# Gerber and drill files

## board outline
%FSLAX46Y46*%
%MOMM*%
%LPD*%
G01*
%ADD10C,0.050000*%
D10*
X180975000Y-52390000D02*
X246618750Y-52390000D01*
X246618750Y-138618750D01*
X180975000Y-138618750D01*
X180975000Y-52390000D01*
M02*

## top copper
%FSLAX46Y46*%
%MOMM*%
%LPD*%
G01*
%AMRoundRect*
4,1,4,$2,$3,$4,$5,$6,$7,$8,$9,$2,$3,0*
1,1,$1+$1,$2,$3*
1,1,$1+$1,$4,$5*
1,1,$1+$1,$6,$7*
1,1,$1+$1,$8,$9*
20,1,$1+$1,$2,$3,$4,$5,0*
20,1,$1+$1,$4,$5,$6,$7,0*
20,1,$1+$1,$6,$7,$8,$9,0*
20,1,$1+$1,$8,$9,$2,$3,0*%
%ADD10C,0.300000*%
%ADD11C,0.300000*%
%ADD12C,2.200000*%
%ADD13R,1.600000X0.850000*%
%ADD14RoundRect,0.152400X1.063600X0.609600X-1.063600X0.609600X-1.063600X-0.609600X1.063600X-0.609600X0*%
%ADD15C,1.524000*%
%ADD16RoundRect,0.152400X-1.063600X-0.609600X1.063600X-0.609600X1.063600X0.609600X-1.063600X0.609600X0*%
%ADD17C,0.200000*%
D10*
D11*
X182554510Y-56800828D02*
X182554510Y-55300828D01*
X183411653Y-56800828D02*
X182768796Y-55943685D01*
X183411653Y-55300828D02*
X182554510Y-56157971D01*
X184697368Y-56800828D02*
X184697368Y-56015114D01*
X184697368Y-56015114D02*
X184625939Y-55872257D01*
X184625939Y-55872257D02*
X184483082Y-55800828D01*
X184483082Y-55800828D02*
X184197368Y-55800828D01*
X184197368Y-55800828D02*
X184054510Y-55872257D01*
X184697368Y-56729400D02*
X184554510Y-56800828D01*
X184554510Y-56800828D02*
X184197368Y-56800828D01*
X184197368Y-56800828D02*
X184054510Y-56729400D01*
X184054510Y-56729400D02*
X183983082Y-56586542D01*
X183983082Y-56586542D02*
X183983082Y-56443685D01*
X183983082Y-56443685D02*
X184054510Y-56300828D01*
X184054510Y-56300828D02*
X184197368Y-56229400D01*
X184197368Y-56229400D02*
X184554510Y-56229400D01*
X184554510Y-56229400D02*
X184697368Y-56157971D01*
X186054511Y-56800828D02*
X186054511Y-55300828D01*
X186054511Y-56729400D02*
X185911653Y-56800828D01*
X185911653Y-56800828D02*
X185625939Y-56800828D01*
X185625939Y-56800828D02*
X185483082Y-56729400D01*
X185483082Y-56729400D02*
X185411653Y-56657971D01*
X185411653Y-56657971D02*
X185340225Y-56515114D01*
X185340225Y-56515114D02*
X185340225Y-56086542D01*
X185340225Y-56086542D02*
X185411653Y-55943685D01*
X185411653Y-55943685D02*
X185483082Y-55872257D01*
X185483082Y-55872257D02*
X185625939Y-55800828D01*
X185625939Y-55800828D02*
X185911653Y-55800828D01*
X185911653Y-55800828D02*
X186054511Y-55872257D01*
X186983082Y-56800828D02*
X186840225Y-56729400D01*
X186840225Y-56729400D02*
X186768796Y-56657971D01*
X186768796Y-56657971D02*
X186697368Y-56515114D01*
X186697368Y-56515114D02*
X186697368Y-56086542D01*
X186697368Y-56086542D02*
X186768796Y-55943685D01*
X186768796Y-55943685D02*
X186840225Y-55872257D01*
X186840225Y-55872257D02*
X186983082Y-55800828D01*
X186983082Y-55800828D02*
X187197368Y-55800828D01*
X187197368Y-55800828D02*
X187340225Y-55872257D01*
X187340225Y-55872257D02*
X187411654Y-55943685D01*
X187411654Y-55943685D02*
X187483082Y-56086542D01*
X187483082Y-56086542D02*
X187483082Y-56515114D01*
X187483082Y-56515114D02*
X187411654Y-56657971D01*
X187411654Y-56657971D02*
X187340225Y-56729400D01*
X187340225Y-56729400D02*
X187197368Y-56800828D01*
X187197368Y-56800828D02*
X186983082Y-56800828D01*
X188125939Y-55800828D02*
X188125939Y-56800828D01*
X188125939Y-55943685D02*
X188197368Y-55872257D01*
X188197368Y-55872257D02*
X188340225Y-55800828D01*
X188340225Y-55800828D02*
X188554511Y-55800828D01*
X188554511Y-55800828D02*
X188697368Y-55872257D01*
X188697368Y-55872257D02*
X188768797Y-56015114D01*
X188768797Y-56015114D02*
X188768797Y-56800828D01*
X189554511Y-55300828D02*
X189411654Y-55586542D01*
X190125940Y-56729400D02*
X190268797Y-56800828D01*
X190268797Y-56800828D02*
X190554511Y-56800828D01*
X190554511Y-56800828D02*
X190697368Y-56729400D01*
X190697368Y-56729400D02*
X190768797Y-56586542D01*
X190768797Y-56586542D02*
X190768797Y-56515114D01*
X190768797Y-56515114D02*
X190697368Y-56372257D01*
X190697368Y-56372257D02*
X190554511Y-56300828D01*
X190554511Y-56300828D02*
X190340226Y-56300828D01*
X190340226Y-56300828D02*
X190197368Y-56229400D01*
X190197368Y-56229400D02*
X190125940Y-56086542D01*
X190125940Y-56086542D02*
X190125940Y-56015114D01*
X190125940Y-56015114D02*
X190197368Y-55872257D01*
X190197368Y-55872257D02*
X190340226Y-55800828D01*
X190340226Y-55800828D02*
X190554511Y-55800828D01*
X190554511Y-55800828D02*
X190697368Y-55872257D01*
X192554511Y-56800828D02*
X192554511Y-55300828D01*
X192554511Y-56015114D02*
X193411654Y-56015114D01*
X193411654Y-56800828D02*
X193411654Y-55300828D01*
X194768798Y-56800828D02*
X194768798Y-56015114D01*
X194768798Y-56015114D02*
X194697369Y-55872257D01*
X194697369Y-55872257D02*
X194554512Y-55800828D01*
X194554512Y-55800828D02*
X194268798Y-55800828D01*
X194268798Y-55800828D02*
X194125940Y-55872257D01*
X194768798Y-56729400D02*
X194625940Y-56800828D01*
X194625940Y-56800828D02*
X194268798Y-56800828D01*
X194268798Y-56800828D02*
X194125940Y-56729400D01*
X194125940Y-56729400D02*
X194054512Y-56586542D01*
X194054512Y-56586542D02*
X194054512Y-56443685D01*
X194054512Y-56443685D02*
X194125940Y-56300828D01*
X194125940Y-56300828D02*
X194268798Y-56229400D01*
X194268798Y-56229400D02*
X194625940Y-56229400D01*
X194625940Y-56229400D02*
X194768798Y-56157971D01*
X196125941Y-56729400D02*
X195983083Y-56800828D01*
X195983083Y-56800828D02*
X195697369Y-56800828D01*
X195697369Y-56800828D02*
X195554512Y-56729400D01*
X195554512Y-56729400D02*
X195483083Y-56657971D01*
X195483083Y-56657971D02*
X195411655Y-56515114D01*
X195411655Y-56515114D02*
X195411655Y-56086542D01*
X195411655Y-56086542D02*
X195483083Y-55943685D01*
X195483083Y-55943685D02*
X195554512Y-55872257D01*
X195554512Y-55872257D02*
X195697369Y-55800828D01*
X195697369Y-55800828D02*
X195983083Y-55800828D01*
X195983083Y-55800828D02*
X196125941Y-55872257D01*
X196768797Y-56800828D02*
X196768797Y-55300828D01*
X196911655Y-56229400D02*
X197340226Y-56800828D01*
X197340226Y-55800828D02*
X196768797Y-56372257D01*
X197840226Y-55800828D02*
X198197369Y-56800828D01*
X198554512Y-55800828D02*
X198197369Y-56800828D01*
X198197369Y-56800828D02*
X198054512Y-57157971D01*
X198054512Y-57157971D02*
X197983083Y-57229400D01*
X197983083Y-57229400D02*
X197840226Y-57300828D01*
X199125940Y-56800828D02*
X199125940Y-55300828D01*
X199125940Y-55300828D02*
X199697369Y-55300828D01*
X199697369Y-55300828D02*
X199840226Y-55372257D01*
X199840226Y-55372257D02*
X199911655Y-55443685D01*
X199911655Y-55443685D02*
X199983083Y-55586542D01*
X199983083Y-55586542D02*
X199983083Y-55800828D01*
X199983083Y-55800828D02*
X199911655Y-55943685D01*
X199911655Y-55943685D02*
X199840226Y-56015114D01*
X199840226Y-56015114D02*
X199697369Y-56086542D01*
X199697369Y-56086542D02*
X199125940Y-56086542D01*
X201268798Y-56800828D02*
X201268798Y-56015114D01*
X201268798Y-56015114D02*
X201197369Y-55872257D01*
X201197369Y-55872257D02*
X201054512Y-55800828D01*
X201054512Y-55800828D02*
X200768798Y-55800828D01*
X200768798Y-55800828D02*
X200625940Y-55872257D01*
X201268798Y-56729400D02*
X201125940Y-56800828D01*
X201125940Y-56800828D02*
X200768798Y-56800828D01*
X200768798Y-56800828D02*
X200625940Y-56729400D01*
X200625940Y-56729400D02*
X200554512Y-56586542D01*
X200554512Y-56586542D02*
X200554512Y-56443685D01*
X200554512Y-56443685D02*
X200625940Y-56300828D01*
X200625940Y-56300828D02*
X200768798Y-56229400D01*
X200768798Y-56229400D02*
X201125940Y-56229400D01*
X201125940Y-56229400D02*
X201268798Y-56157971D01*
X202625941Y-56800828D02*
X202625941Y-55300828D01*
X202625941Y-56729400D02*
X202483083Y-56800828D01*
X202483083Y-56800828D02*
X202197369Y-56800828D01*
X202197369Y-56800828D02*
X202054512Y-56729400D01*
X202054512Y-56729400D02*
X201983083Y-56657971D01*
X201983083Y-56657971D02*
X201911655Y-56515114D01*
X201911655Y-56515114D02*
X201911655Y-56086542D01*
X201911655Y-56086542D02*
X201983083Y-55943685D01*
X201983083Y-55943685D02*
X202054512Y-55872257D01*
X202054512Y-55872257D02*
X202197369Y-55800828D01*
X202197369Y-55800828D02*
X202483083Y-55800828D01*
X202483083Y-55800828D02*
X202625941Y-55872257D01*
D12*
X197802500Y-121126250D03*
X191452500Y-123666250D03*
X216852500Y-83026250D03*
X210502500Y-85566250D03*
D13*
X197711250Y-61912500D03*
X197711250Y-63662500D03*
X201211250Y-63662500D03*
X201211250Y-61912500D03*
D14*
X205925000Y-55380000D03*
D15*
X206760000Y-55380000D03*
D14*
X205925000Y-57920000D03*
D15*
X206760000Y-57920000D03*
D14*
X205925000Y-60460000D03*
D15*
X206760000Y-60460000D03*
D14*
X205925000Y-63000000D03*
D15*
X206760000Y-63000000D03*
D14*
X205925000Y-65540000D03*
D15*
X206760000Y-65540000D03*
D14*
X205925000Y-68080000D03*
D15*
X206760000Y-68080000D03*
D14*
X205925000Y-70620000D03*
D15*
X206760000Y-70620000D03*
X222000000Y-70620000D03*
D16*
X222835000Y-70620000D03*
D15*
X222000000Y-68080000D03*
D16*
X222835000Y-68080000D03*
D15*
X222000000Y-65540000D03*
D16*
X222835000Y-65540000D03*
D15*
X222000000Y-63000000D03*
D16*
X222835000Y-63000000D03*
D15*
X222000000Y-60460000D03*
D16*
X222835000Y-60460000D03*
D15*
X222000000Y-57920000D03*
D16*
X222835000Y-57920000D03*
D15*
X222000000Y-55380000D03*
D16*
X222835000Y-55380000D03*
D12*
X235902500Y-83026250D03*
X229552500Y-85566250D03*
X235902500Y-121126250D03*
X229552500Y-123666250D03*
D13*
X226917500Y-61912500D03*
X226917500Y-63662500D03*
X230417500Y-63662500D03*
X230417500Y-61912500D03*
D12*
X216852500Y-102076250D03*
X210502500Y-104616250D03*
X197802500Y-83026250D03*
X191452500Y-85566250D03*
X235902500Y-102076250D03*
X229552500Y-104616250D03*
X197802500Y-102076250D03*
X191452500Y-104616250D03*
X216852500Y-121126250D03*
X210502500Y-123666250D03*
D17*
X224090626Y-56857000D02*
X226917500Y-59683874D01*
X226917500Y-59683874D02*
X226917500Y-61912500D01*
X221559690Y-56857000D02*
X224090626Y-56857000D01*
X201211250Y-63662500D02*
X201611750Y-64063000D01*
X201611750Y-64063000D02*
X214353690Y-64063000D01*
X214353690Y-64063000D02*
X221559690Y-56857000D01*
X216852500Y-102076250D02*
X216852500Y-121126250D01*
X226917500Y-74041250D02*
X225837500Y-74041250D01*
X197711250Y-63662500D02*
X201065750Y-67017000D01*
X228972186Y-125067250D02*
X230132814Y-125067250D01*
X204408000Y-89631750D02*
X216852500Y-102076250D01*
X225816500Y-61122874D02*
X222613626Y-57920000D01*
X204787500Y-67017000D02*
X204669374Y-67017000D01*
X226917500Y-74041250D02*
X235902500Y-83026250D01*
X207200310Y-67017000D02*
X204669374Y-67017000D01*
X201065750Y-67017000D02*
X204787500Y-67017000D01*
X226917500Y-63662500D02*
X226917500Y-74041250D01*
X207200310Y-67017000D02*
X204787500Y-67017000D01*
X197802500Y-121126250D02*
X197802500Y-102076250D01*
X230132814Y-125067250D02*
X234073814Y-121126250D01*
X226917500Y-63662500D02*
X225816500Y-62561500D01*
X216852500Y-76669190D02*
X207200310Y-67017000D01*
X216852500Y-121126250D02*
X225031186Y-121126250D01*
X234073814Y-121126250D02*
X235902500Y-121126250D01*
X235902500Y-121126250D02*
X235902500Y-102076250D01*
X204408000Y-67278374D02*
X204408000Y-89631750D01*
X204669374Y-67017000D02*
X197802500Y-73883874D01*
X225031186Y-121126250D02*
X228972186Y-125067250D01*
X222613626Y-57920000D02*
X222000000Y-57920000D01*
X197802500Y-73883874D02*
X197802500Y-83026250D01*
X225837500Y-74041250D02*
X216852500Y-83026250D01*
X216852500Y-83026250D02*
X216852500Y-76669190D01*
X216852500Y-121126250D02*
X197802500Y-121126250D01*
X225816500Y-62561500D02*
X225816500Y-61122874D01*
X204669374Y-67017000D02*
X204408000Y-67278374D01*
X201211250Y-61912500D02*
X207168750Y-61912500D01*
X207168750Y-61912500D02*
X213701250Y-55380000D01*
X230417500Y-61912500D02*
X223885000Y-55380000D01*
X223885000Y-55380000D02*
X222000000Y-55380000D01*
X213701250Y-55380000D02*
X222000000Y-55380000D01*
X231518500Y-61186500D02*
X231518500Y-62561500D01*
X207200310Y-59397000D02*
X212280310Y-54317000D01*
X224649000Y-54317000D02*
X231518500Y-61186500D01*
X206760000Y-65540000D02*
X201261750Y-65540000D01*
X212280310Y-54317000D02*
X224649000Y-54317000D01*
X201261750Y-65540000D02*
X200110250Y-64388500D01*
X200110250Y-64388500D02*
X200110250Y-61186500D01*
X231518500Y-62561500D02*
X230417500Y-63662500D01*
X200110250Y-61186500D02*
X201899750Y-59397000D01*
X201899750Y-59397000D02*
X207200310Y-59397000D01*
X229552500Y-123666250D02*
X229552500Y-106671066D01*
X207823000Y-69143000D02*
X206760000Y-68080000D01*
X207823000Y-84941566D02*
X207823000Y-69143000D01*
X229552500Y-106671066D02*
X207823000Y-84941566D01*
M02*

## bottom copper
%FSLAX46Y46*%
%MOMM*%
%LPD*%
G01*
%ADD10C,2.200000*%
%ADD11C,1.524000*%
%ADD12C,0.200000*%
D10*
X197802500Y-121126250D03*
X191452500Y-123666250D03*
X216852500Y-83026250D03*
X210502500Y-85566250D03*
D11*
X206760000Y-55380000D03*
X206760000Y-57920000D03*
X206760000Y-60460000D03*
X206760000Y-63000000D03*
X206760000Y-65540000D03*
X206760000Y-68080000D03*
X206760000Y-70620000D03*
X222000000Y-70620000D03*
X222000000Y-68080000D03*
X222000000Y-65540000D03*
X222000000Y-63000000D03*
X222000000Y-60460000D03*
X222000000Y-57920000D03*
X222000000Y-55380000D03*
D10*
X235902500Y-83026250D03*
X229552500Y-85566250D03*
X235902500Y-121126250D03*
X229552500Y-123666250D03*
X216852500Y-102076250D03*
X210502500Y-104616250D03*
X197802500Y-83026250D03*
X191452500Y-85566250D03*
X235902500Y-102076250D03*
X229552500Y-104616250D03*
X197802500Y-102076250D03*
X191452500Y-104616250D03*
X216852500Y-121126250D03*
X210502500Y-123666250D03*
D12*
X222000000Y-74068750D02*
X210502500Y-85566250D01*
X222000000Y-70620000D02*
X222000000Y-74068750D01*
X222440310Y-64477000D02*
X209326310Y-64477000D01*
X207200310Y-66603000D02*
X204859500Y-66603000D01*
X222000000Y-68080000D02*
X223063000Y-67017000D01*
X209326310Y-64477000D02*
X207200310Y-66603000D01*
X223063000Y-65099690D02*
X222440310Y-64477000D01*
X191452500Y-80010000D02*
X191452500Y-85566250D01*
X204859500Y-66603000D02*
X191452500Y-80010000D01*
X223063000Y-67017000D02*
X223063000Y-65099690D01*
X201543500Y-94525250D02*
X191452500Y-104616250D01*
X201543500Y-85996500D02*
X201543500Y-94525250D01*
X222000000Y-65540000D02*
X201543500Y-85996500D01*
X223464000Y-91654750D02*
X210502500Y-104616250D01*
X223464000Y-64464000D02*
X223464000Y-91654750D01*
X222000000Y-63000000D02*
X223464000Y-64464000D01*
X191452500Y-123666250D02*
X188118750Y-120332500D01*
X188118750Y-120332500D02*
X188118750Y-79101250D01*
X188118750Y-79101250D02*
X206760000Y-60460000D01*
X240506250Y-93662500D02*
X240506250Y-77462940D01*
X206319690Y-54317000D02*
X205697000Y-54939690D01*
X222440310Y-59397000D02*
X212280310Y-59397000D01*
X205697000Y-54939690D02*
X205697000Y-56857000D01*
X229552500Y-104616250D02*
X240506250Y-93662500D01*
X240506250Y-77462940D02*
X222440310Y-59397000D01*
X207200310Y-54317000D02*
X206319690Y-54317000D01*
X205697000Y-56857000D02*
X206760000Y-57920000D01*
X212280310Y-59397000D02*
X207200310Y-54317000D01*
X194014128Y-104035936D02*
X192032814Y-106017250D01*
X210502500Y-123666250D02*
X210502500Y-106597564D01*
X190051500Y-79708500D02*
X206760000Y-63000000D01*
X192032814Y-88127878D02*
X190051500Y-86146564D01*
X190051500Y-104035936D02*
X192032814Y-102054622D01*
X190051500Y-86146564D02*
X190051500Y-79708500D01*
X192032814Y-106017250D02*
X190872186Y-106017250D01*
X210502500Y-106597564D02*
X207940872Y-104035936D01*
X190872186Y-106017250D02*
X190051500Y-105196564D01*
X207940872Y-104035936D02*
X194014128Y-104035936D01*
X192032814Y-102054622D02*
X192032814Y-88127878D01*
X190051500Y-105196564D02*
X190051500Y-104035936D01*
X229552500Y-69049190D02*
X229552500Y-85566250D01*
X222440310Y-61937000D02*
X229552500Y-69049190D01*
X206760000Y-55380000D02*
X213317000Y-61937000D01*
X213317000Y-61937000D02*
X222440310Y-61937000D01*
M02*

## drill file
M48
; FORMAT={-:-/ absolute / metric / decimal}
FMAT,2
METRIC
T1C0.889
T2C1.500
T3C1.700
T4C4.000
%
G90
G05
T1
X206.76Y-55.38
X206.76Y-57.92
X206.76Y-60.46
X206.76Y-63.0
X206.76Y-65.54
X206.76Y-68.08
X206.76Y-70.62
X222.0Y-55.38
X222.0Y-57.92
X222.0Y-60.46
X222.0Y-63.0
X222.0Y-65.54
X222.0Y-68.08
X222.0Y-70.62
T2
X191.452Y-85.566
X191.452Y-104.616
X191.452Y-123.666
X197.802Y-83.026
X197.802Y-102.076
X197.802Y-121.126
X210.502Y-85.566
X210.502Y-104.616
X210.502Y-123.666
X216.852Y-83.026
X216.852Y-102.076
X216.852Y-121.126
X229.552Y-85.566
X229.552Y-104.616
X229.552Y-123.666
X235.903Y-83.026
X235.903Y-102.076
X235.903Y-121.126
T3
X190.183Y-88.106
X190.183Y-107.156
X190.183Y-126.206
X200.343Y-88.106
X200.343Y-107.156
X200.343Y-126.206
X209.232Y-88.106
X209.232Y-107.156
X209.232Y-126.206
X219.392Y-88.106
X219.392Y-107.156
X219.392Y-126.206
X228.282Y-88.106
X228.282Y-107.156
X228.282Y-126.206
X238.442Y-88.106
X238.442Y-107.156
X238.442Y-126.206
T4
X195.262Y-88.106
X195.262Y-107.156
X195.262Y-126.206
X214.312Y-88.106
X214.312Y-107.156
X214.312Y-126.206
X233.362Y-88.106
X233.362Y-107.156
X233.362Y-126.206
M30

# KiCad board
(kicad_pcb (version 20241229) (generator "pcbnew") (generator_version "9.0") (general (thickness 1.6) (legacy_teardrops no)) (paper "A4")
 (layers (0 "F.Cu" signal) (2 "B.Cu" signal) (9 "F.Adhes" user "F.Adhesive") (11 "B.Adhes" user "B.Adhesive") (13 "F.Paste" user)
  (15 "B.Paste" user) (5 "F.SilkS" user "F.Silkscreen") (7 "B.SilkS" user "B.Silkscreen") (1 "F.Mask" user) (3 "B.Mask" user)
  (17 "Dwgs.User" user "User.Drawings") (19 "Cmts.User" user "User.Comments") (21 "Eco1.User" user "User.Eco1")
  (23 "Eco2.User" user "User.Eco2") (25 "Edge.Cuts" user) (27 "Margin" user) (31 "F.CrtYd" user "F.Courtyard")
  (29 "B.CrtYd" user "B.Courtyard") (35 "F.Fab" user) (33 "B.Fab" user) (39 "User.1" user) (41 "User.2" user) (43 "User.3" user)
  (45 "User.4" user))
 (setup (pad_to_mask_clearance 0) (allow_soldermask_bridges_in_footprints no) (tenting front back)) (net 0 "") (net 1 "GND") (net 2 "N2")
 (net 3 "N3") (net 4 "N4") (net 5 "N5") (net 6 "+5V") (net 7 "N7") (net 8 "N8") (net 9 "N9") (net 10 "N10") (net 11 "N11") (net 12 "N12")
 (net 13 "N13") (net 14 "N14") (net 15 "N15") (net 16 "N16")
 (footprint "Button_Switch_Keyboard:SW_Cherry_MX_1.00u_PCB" (layer "F.Cu") (at 197.8025 121.12625)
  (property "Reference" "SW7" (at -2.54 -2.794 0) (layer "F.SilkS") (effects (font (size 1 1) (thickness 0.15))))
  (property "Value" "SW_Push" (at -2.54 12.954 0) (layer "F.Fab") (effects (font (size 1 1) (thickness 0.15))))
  (pad "" np_thru_hole circle (at -7.62 5.08) (size 1.7 1.7) (drill 1.7) (layers "*.Cu" "*.Mask"))
  (pad "" np_thru_hole circle (at -2.54 5.08) (size 4 4) (drill 4) (layers "*.Cu" "*.Mask"))
  (pad "" np_thru_hole circle (at 2.54 5.08) (size 1.7 1.7) (drill 1.7) (layers "*.Cu" "*.Mask"))
  (pad "1" thru_hole circle (at 0 0) (size 2.2 2.2) (drill 1.5) (layers "*.Cu" "*.Mask") (remove_unused_layers no) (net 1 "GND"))
  (pad "2" thru_hole circle (at -6.35 2.54) (size 2.2 2.2) (drill 1.5) (layers "*.Cu" "*.Mask") (remove_unused_layers no) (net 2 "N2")))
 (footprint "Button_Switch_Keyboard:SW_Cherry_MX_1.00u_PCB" (layer "F.Cu") (at 216.8525 83.02625)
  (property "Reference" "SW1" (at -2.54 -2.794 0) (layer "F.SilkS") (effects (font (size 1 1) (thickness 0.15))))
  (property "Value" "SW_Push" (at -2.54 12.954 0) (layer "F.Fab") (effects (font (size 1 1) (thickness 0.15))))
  (pad "" np_thru_hole circle (at -7.62 5.08) (size 1.7 1.7) (drill 1.7) (layers "*.Cu" "*.Mask"))
  (pad "" np_thru_hole circle (at -2.54 5.08) (size 4 4) (drill 4) (layers "*.Cu" "*.Mask"))
  (pad "" np_thru_hole circle (at 2.54 5.08) (size 1.7 1.7) (drill 1.7) (layers "*.Cu" "*.Mask"))
  (pad "1" thru_hole circle (at 0 0) (size 2.2 2.2) (drill 1.5) (layers "*.Cu" "*.Mask") (remove_unused_layers no) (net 1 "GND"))
  (pad "2" thru_hole circle (at -6.35 2.54) (size 2.2 2.2) (drill 1.5) (layers "*.Cu" "*.Mask") (remove_unused_layers no) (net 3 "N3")))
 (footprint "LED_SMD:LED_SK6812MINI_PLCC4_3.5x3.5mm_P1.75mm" (layer "F.Cu") (at 199.46125 62.7875)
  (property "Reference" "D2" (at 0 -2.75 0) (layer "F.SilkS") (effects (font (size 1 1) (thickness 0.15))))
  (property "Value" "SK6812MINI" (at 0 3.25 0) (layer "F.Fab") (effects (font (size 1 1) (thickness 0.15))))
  (pad "1" smd rect (at -1.75 -0.875) (size 1.6 0.85) (layers "F.Cu" "F.Mask" "F.Paste") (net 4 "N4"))
  (pad "2" smd rect (at -1.75 0.875) (size 1.6 0.85) (layers "F.Cu" "F.Mask" "F.Paste") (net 1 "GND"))
  (pad "3" smd rect (at 1.75 0.875) (size 1.6 0.85) (layers "F.Cu" "F.Mask" "F.Paste") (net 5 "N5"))
  (pad "4" smd rect (at 1.75 -0.875) (size 1.6 0.85) (layers "F.Cu" "F.Mask" "F.Paste") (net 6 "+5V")))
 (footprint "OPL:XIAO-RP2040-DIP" (layer "F.Cu") (at 214.38 63)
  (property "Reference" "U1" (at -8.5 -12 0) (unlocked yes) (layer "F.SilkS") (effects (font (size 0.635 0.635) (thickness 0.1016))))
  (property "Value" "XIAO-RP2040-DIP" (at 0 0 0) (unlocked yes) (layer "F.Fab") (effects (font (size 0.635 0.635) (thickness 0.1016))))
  (pad "1" smd roundrect (at -8.455 -7.62 180) (size 2.432 1.524) (layers "F.Cu" "F.Mask") (roundrect_rratio 0.1) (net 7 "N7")
   (thermal_bridge_angle 45))
  (pad "1" thru_hole circle (at -7.62 -7.62 180) (size 1.524 1.524) (drill 0.889) (layers "*.Cu" "*.Mask") (remove_unused_layers no)
   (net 7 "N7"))
  (pad "2" smd roundrect (at -8.455 -5.08 180) (size 2.432 1.524) (layers "F.Cu" "F.Mask") (roundrect_rratio 0.1) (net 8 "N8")
   (thermal_bridge_angle 45))
  (pad "2" thru_hole circle (at -7.62 -5.08 180) (size 1.524 1.524) (drill 0.889) (layers "*.Cu" "*.Mask") (remove_unused_layers no)
   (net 8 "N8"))
  (pad "3" smd roundrect (at -8.455 -2.54 180) (size 2.432 1.524) (layers "F.Cu" "F.Mask") (roundrect_rratio 0.1) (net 2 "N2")
   (thermal_bridge_angle 45))
  (pad "3" thru_hole circle (at -7.62 -2.54 180) (size 1.524 1.524) (drill 0.889) (layers "*.Cu" "*.Mask") (remove_unused_layers no)
   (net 2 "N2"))
  (pad "4" smd roundrect (at -8.455 0 180) (size 2.432 1.524) (layers "F.Cu" "F.Mask") (roundrect_rratio 0.1) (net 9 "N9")
   (thermal_bridge_angle 45))
  (pad "4" thru_hole circle (at -7.62 0 180) (size 1.524 1.524) (drill 0.889) (layers "*.Cu" "*.Mask") (remove_unused_layers no)
   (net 9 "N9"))
  (pad "5" smd roundrect (at -8.455 2.54 180) (size 2.432 1.524) (layers "F.Cu" "F.Mask") (roundrect_rratio 0.1) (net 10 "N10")
   (thermal_bridge_angle 45))
  (pad "5" thru_hole circle (at -7.62 2.54 180) (size 1.524 1.524) (drill 0.889) (layers "*.Cu" "*.Mask") (remove_unused_layers no)
   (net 10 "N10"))
  (pad "6" smd roundrect (at -8.455 5.08 180) (size 2.432 1.524) (layers "F.Cu" "F.Mask") (roundrect_rratio 0.1) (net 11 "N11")
   (thermal_bridge_angle 45))
  (pad "6" thru_hole circle (at -7.62 5.08 180) (size 1.524 1.524) (drill 0.889) (layers "*.Cu" "*.Mask") (remove_unused_layers no)
   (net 11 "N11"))
  (pad "7" smd roundrect (at -8.455 7.62 180) (size 2.432 1.524) (layers "F.Cu" "F.Mask") (roundrect_rratio 0.1) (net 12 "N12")
   (thermal_bridge_angle 45))
  (pad "7" thru_hole circle (at -7.62 7.62 180) (size 1.524 1.524) (drill 0.889) (layers "*.Cu" "*.Mask") (remove_unused_layers no)
   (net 12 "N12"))
  (pad "8" thru_hole circle (at 7.62 7.62) (size 1.524 1.524) (drill 0.889) (layers "*.Cu" "*.Mask") (remove_unused_layers no) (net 3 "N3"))
  (pad "8" smd roundrect (at 8.455 7.62) (size 2.432 1.524) (layers "F.Cu" "F.Mask") (roundrect_rratio 0.1) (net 3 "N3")
   (thermal_bridge_angle 45))
  (pad "9" thru_hole circle (at 7.62 5.08) (size 1.524 1.524) (drill 0.889) (layers "*.Cu" "*.Mask") (remove_unused_layers no)
   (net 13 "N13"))
  (pad "9" smd roundrect (at 8.455 5.08) (size 2.432 1.524) (layers "F.Cu" "F.Mask") (roundrect_rratio 0.1) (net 13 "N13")
   (thermal_bridge_angle 45))
  (pad "10" thru_hole circle (at 7.62 2.54) (size 1.524 1.524) (drill 0.889) (layers "*.Cu" "*.Mask") (remove_unused_layers no)
   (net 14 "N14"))
  (pad "10" smd roundrect (at 8.455 2.54) (size 2.432 1.524) (layers "F.Cu" "F.Mask") (roundrect_rratio 0.1) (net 14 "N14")
   (thermal_bridge_angle 45))
  (pad "11" thru_hole circle (at 7.62 0) (size 1.524 1.524) (drill 0.889) (layers "*.Cu" "*.Mask") (remove_unused_layers no) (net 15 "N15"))
  (pad "11" smd roundrect (at 8.455 0) (size 2.432 1.524) (layers "F.Cu" "F.Mask") (roundrect_rratio 0.1) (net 15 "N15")
   (thermal_bridge_angle 45))
  (pad "12" thru_hole circle (at 7.62 -2.54) (size 1.524 1.524) (drill 0.889) (layers "*.Cu" "*.Mask") (remove_unused_layers no)
   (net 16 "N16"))
  (pad "12" smd roundrect (at 8.455 -2.54) (size 2.432 1.524) (layers "F.Cu" "F.Mask") (roundrect_rratio 0.1) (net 16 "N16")
   (thermal_bridge_angle 45))
  (pad "13" thru_hole circle (at 7.62 -5.08) (size 1.524 1.524) (drill 0.889) (layers "*.Cu" "*.Mask") (remove_unused_layers no)
   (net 1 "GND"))
  (pad "13" smd roundrect (at 8.455 -5.08) (size 2.432 1.524) (layers "F.Cu" "F.Mask") (roundrect_rratio 0.1) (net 1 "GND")
   (thermal_bridge_angle 45))
  (pad "14" thru_hole circle (at 7.62 -7.62) (size 1.524 1.524) (drill 0.889) (layers "*.Cu" "*.Mask") (remove_unused_layers no)
   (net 6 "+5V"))
  (pad "14" smd roundrect (at 8.455 -7.62) (size 2.432 1.524) (layers "F.Cu" "F.Mask") (roundrect_rratio 0.1) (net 6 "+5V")
   (thermal_bridge_angle 45)))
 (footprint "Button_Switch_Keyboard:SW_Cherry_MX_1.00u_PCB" (layer "F.Cu") (at 235.9025 83.02625)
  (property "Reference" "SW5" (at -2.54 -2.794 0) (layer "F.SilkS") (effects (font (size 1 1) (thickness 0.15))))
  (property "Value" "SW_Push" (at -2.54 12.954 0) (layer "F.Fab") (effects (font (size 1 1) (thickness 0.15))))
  (pad "" np_thru_hole circle (at -7.62 5.08) (size 1.7 1.7) (drill 1.7) (layers "*.Cu" "*.Mask"))
  (pad "" np_thru_hole circle (at -2.54 5.08) (size 4 4) (drill 4) (layers "*.Cu" "*.Mask"))
  (pad "" np_thru_hole circle (at 2.54 5.08) (size 1.7 1.7) (drill 1.7) (layers "*.Cu" "*.Mask"))
  (pad "1" thru_hole circle (at 0 0) (size 2.2 2.2) (drill 1.5) (layers "*.Cu" "*.Mask") (remove_unused_layers no) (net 1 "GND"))
  (pad "2" thru_hole circle (at -6.35 2.54) (size 2.2 2.2) (drill 1.5) (layers "*.Cu" "*.Mask") (remove_unused_layers no) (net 7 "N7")))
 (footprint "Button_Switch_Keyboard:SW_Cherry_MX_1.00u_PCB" (layer "F.Cu") (at 235.9025 121.12625)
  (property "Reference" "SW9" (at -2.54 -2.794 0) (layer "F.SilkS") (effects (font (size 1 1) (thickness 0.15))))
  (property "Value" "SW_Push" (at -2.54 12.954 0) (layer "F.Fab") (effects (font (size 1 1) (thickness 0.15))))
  (pad "" np_thru_hole circle (at -7.62 5.08) (size 1.7 1.7) (drill 1.7) (layers "*.Cu" "*.Mask"))
  (pad "" np_thru_hole circle (at -2.54 5.08) (size 4 4) (drill 4) (layers "*.Cu" "*.Mask"))
  (pad "" np_thru_hole circle (at 2.54 5.08) (size 1.7 1.7) (drill 1.7) (layers "*.Cu" "*.Mask"))
  (pad "1" thru_hole circle (at 0 0) (size 2.2 2.2) (drill 1.5) (layers "*.Cu" "*.Mask") (remove_unused_layers no) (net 1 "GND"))
  (pad "2" thru_hole circle (at -6.35 2.54) (size 2.2 2.2) (drill 1.5) (layers "*.Cu" "*.Mask") (remove_unused_layers no) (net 11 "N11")))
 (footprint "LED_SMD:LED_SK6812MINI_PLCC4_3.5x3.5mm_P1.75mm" (layer "F.Cu") (at 228.6675 62.7875)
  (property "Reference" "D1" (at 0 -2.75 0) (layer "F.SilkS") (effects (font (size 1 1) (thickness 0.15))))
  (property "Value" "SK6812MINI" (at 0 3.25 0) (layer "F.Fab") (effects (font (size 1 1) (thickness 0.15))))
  (pad "1" smd rect (at -1.75 -0.875) (size 1.6 0.85) (layers "F.Cu" "F.Mask" "F.Paste") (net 5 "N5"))
  (pad "2" smd rect (at -1.75 0.875) (size 1.6 0.85) (layers "F.Cu" "F.Mask" "F.Paste") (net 1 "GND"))
  (pad "3" smd rect (at 1.75 0.875) (size 1.6 0.85) (layers "F.Cu" "F.Mask" "F.Paste") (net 10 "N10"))
  (pad "4" smd rect (at 1.75 -0.875) (size 1.6 0.85) (layers "F.Cu" "F.Mask" "F.Paste") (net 6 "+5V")))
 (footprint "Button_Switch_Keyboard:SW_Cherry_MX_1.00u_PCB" (layer "F.Cu") (at 216.8525 102.07625)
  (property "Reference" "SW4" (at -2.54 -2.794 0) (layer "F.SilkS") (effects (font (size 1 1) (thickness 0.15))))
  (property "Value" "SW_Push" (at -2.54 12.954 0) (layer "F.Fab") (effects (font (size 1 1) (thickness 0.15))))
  (pad "" np_thru_hole circle (at -7.62 5.08) (size 1.7 1.7) (drill 1.7) (layers "*.Cu" "*.Mask"))
  (pad "" np_thru_hole circle (at -2.54 5.08) (size 4 4) (drill 4) (layers "*.Cu" "*.Mask"))
  (pad "" np_thru_hole circle (at 2.54 5.08) (size 1.7 1.7) (drill 1.7) (layers "*.Cu" "*.Mask"))
  (pad "1" thru_hole circle (at 0 0) (size 2.2 2.2) (drill 1.5) (layers "*.Cu" "*.Mask") (remove_unused_layers no) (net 1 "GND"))
  (pad "2" thru_hole circle (at -6.35 2.54) (size 2.2 2.2) (drill 1.5) (layers "*.Cu" "*.Mask") (remove_unused_layers no) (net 15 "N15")))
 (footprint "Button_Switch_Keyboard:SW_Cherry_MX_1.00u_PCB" (layer "F.Cu") (at 197.8025 83.02625)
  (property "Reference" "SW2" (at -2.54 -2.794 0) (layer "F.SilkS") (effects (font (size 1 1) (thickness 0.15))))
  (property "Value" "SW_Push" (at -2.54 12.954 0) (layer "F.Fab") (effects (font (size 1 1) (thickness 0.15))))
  (pad "" np_thru_hole circle (at -7.62 5.08) (size 1.7 1.7) (drill 1.7) (layers "*.Cu" "*.Mask"))
  (pad "" np_thru_hole circle (at -2.54 5.08) (size 4 4) (drill 4) (layers "*.Cu" "*.Mask"))
  (pad "" np_thru_hole circle (at 2.54 5.08) (size 1.7 1.7) (drill 1.7) (layers "*.Cu" "*.Mask"))
  (pad "1" thru_hole circle (at 0 0) (size 2.2 2.2) (drill 1.5) (layers "*.Cu" "*.Mask") (remove_unused_layers no) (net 1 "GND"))
  (pad "2" thru_hole circle (at -6.35 2.54) (size 2.2 2.2) (drill 1.5) (layers "*.Cu" "*.Mask") (remove_unused_layers no) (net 13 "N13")))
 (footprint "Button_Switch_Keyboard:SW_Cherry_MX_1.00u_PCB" (layer "F.Cu") (at 235.9025 102.07625)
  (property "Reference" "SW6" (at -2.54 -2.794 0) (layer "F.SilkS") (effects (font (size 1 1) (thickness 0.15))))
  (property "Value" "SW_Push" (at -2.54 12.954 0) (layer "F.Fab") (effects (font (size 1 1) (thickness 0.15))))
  (pad "" np_thru_hole circle (at -7.62 5.08) (size 1.7 1.7) (drill 1.7) (layers "*.Cu" "*.Mask"))
  (pad "" np_thru_hole circle (at -2.54 5.08) (size 4 4) (drill 4) (layers "*.Cu" "*.Mask"))
  (pad "" np_thru_hole circle (at 2.54 5.08) (size 1.7 1.7) (drill 1.7) (layers "*.Cu" "*.Mask"))
  (pad "1" thru_hole circle (at 0 0) (size 2.2 2.2) (drill 1.5) (layers "*.Cu" "*.Mask") (remove_unused_layers no) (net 1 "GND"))
  (pad "2" thru_hole circle (at -6.35 2.54) (size 2.2 2.2) (drill 1.5) (layers "*.Cu" "*.Mask") (remove_unused_layers no) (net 8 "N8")))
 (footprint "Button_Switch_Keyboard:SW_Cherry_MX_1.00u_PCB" (layer "F.Cu") (at 197.8025 102.07625)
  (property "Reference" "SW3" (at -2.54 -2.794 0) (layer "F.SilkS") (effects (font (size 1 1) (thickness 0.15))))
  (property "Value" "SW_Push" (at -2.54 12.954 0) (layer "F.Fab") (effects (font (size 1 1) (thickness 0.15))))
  (pad "" np_thru_hole circle (at -7.62 5.08) (size 1.7 1.7) (drill 1.7) (layers "*.Cu" "*.Mask"))
  (pad "" np_thru_hole circle (at -2.54 5.08) (size 4 4) (drill 4) (layers "*.Cu" "*.Mask"))
  (pad "" np_thru_hole circle (at 2.54 5.08) (size 1.7 1.7) (drill 1.7) (layers "*.Cu" "*.Mask"))
  (pad "1" thru_hole circle (at 0 0) (size 2.2 2.2) (drill 1.5) (layers "*.Cu" "*.Mask") (remove_unused_layers no) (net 1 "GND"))
  (pad "2" thru_hole circle (at -6.35 2.54) (size 2.2 2.2) (drill 1.5) (layers "*.Cu" "*.Mask") (remove_unused_layers no) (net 14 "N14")))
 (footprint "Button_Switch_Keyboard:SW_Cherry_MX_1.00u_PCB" (layer "F.Cu") (at 216.8525 121.12625)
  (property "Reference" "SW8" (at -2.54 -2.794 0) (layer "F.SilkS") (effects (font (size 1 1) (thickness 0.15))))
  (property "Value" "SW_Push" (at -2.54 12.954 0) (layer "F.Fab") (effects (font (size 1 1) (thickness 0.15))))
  (pad "" np_thru_hole circle (at -7.62 5.08) (size 1.7 1.7) (drill 1.7) (layers "*.Cu" "*.Mask"))
  (pad "" np_thru_hole circle (at -2.54 5.08) (size 4 4) (drill 4) (layers "*.Cu" "*.Mask"))
  (pad "" np_thru_hole circle (at 2.54 5.08) (size 1.7 1.7) (drill 1.7) (layers "*.Cu" "*.Mask"))
  (pad "1" thru_hole circle (at 0 0) (size 2.2 2.2) (drill 1.5) (layers "*.Cu" "*.Mask") (remove_unused_layers no) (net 1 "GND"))
  (pad "2" thru_hole circle (at -6.35 2.54) (size 2.2 2.2) (drill 1.5) (layers "*.Cu" "*.Mask") (remove_unused_layers no) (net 9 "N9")))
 (gr_rect (start 180.975 52.39) (end 246.61875 138.61875) (stroke (width 0.05) (type default)) (fill no) (layer "Edge.Cuts"))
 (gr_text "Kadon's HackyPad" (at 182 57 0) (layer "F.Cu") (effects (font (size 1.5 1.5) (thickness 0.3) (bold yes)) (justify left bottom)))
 (segment (start 224.090626 56.857) (end 226.9175 59.683874) (width 0.2) (layer "F.Cu") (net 5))
 (segment (start 226.9175 59.683874) (end 226.9175 61.9125) (width 0.2) (layer "F.Cu") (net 5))
 (segment (start 221.55969 56.857) (end 224.090626 56.857) (width 0.2) (layer "F.Cu") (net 5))
 (segment (start 201.21125 63.6625) (end 201.61175 64.063) (width 0.2) (layer "F.Cu") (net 5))
 (segment (start 201.61175 64.063) (end 214.35369 64.063) (width 0.2) (layer "F.Cu") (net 5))
 (segment (start 214.35369 64.063) (end 221.55969 56.857) (width 0.2) (layer "F.Cu") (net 5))
 (segment (start 216.8525 102.07625) (end 216.8525 121.12625) (width 0.2) (layer "F.Cu") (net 1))
 (segment (start 226.9175 74.04125) (end 225.8375 74.04125) (width 0.2) (layer "F.Cu") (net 1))
 (segment (start 197.71125 63.6625) (end 201.06575 67.017) (width 0.2) (layer "F.Cu") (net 1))
 (segment (start 228.972186 125.06725) (end 230.132814 125.06725) (width 0.2) (layer "F.Cu") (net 1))
 (segment (start 204.408 89.63175) (end 216.8525 102.07625) (width 0.2) (layer "F.Cu") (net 1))
 (segment (start 225.8165 61.122874) (end 222.613626 57.92) (width 0.2) (layer "F.Cu") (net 1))
 (segment (start 204.7875 67.017) (end 204.669374 67.017) (width 0.2) (layer "F.Cu") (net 1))
 (segment (start 226.9175 74.04125) (end 235.9025 83.02625) (width 0.2) (layer "F.Cu") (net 1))
 (segment (start 207.20031 67.017) (end 204.669374 67.017) (width 0.2) (layer "F.Cu") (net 1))
 (segment (start 201.06575 67.017) (end 204.7875 67.017) (width 0.2) (layer "F.Cu") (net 1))
 (segment (start 226.9175 63.6625) (end 226.9175 74.04125) (width 0.2) (layer "F.Cu") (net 1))
 (segment (start 207.20031 67.017) (end 204.7875 67.017) (width 0.2) (layer "F.Cu") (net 1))
 (segment (start 197.8025 121.12625) (end 197.8025 102.07625) (width 0.2) (layer "F.Cu") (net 1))
 (segment (start 230.132814 125.06725) (end 234.073814 121.12625) (width 0.2) (layer "F.Cu") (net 1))
 (segment (start 226.9175 63.6625) (end 225.8165 62.5615) (width 0.2) (layer "F.Cu") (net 1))
 (segment (start 216.8525 76.66919) (end 207.20031 67.017) (width 0.2) (layer "F.Cu") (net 1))
 (segment (start 216.8525 121.12625) (end 225.031186 121.12625) (width 0.2) (layer "F.Cu") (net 1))
 (segment (start 234.073814 121.12625) (end 235.9025 121.12625) (width 0.2) (layer "F.Cu") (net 1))
 (segment (start 235.9025 121.12625) (end 235.9025 102.07625) (width 0.2) (layer "F.Cu") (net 1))
 (segment (start 204.408 67.278374) (end 204.408 89.63175) (width 0.2) (layer "F.Cu") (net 1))
 (segment (start 204.669374 67.017) (end 197.8025 73.883874) (width 0.2) (layer "F.Cu") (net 1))
 (segment (start 225.031186 121.12625) (end 228.972186 125.06725) (width 0.2) (layer "F.Cu") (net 1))
 (segment (start 222.613626 57.92) (end 222 57.92) (width 0.2) (layer "F.Cu") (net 1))
 (segment (start 197.8025 73.883874) (end 197.8025 83.02625) (width 0.2) (layer "F.Cu") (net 1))
 (segment (start 225.8375 74.04125) (end 216.8525 83.02625) (width 0.2) (layer "F.Cu") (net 1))
 (segment (start 216.8525 83.02625) (end 216.8525 76.66919) (width 0.2) (layer "F.Cu") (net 1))
 (segment (start 216.8525 121.12625) (end 197.8025 121.12625) (width 0.2) (layer "F.Cu") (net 1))
 (segment (start 225.8165 62.5615) (end 225.8165 61.122874) (width 0.2) (layer "F.Cu") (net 1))
 (segment (start 204.669374 67.017) (end 204.408 67.278374) (width 0.2) (layer "F.Cu") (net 1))
 (segment (start 201.21125 61.9125) (end 207.16875 61.9125) (width 0.2) (layer "F.Cu") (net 6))
 (segment (start 207.16875 61.9125) (end 213.70125 55.38) (width 0.2) (layer "F.Cu") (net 6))
 (segment (start 230.4175 61.9125) (end 223.885 55.38) (width 0.2) (layer "F.Cu") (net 6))
 (segment (start 223.885 55.38) (end 222 55.38) (width 0.2) (layer "F.Cu") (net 6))
 (segment (start 213.70125 55.38) (end 222 55.38) (width 0.2) (layer "F.Cu") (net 6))
 (segment (start 231.5185 61.1865) (end 231.5185 62.5615) (width 0.2) (layer "F.Cu") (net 10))
 (segment (start 207.20031 59.397) (end 212.28031 54.317) (width 0.2) (layer "F.Cu") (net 10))
 (segment (start 224.649 54.317) (end 231.5185 61.1865) (width 0.2) (layer "F.Cu") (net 10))
 (segment (start 206.76 65.54) (end 201.26175 65.54) (width 0.2) (layer "F.Cu") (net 10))
 (segment (start 212.28031 54.317) (end 224.649 54.317) (width 0.2) (layer "F.Cu") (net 10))
 (segment (start 201.26175 65.54) (end 200.11025 64.3885) (width 0.2) (layer "F.Cu") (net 10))
 (segment (start 200.11025 64.3885) (end 200.11025 61.1865) (width 0.2) (layer "F.Cu") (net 10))
 (segment (start 231.5185 62.5615) (end 230.4175 63.6625) (width 0.2) (layer "F.Cu") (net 10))
 (segment (start 200.11025 61.1865) (end 201.89975 59.397) (width 0.2) (layer "F.Cu") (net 10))
 (segment (start 201.89975 59.397) (end 207.20031 59.397) (width 0.2) (layer "F.Cu") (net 10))
 (segment (start 222 74.06875) (end 210.5025 85.56625) (width 0.2) (layer "B.Cu") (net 3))
 (segment (start 222 70.62) (end 222 74.06875) (width 0.2) (layer "B.Cu") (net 3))
 (segment (start 222.44031 64.477) (end 209.32631 64.477) (width 0.2) (layer "B.Cu") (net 13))
 (segment (start 207.20031 66.603) (end 204.8595 66.603) (width 0.2) (layer "B.Cu") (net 13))
 (segment (start 222 68.08) (end 223.063 67.017) (width 0.2) (layer "B.Cu") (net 13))
 (segment (start 209.32631 64.477) (end 207.20031 66.603) (width 0.2) (layer "B.Cu") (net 13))
 (segment (start 223.063 65.09969) (end 222.44031 64.477) (width 0.2) (layer "B.Cu") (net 13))
 (segment (start 191.4525 80.01) (end 191.4525 85.56625) (width 0.2) (layer "B.Cu") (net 13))
 (segment (start 204.8595 66.603) (end 191.4525 80.01) (width 0.2) (layer "B.Cu") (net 13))
 (segment (start 223.063 67.017) (end 223.063 65.09969) (width 0.2) (layer "B.Cu") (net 13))
 (segment (start 201.5435 94.52525) (end 191.4525 104.61625) (width 0.2) (layer "B.Cu") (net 14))
 (segment (start 201.5435 85.9965) (end 201.5435 94.52525) (width 0.2) (layer "B.Cu") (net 14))
 (segment (start 222 65.54) (end 201.5435 85.9965) (width 0.2) (layer "B.Cu") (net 14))
 (segment (start 223.464 91.65475) (end 210.5025 104.61625) (width 0.2) (layer "B.Cu") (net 15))
 (segment (start 223.464 64.464) (end 223.464 91.65475) (width 0.2) (layer "B.Cu") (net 15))
 (segment (start 222 63) (end 223.464 64.464) (width 0.2) (layer "B.Cu") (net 15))
 (segment (start 191.4525 123.66625) (end 188.11875 120.3325) (width 0.2) (layer "B.Cu") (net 2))
 (segment (start 188.11875 120.3325) (end 188.11875 79.10125) (width 0.2) (layer "B.Cu") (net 2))
 (segment (start 188.11875 79.10125) (end 206.76 60.46) (width 0.2) (layer "B.Cu") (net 2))
 (segment (start 229.5525 123.66625) (end 229.5525 106.671066) (width 0.2) (layer "F.Cu") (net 11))
 (segment (start 207.823 69.143) (end 206.76 68.08) (width 0.2) (layer "F.Cu") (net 11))
 (segment (start 207.823 84.941566) (end 207.823 69.143) (width 0.2) (layer "F.Cu") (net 11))
 (segment (start 229.5525 106.671066) (end 207.823 84.941566) (width 0.2) (layer "F.Cu") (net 11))
 (segment (start 240.50625 93.6625) (end 240.50625 77.46294) (width 0.2) (layer "B.Cu") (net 8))
 (segment (start 206.31969 54.317) (end 205.697 54.93969) (width 0.2) (layer "B.Cu") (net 8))
 (segment (start 222.44031 59.397) (end 212.28031 59.397) (width 0.2) (layer "B.Cu") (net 8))
 (segment (start 205.697 54.93969) (end 205.697 56.857) (width 0.2) (layer "B.Cu") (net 8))
 (segment (start 229.5525 104.61625) (end 240.50625 93.6625) (width 0.2) (layer "B.Cu") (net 8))
 (segment (start 240.50625 77.46294) (end 222.44031 59.397) (width 0.2) (layer "B.Cu") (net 8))
 (segment (start 207.20031 54.317) (end 206.31969 54.317) (width 0.2) (layer "B.Cu") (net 8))
 (segment (start 205.697 56.857) (end 206.76 57.92) (width 0.2) (layer "B.Cu") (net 8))
 (segment (start 212.28031 59.397) (end 207.20031 54.317) (width 0.2) (layer "B.Cu") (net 8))
 (segment (start 194.014128 104.035936) (end 192.032814 106.01725) (width 0.2) (layer "B.Cu") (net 9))
 (segment (start 210.5025 123.66625) (end 210.5025 106.597564) (width 0.2) (layer "B.Cu") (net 9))
 (segment (start 190.0515 79.7085) (end 206.76 63) (width 0.2) (layer "B.Cu") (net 9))
 (segment (start 192.032814 88.127878) (end 190.0515 86.146564) (width 0.2) (layer "B.Cu") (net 9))
 (segment (start 190.0515 104.035936) (end 192.032814 102.054622) (width 0.2) (layer "B.Cu") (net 9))
 (segment (start 190.0515 86.146564) (end 190.0515 79.7085) (width 0.2) (layer "B.Cu") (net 9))
 (segment (start 192.032814 106.01725) (end 190.872186 106.01725) (width 0.2) (layer "B.Cu") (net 9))
 (segment (start 210.5025 106.597564) (end 207.940872 104.035936) (width 0.2) (layer "B.Cu") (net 9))
 (segment (start 190.872186 106.01725) (end 190.0515 105.196564) (width 0.2) (layer "B.Cu") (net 9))
 (segment (start 207.940872 104.035936) (end 194.014128 104.035936) (width 0.2) (layer "B.Cu") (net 9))
 (segment (start 192.032814 102.054622) (end 192.032814 88.127878) (width 0.2) (layer "B.Cu") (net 9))
 (segment (start 190.0515 105.196564) (end 190.0515 104.035936) (width 0.2) (layer "B.Cu") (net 9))
 (segment (start 229.5525 69.04919) (end 229.5525 85.56625) (width 0.2) (layer "B.Cu") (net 7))
 (segment (start 222.44031 61.937) (end 229.5525 69.04919) (width 0.2) (layer "B.Cu") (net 7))
 (segment (start 206.76 55.38) (end 213.317 61.937) (width 0.2) (layer "B.Cu") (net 7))
 (segment (start 213.317 61.937) (end 222.44031 61.937) (width 0.2) (layer "B.Cu") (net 7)))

